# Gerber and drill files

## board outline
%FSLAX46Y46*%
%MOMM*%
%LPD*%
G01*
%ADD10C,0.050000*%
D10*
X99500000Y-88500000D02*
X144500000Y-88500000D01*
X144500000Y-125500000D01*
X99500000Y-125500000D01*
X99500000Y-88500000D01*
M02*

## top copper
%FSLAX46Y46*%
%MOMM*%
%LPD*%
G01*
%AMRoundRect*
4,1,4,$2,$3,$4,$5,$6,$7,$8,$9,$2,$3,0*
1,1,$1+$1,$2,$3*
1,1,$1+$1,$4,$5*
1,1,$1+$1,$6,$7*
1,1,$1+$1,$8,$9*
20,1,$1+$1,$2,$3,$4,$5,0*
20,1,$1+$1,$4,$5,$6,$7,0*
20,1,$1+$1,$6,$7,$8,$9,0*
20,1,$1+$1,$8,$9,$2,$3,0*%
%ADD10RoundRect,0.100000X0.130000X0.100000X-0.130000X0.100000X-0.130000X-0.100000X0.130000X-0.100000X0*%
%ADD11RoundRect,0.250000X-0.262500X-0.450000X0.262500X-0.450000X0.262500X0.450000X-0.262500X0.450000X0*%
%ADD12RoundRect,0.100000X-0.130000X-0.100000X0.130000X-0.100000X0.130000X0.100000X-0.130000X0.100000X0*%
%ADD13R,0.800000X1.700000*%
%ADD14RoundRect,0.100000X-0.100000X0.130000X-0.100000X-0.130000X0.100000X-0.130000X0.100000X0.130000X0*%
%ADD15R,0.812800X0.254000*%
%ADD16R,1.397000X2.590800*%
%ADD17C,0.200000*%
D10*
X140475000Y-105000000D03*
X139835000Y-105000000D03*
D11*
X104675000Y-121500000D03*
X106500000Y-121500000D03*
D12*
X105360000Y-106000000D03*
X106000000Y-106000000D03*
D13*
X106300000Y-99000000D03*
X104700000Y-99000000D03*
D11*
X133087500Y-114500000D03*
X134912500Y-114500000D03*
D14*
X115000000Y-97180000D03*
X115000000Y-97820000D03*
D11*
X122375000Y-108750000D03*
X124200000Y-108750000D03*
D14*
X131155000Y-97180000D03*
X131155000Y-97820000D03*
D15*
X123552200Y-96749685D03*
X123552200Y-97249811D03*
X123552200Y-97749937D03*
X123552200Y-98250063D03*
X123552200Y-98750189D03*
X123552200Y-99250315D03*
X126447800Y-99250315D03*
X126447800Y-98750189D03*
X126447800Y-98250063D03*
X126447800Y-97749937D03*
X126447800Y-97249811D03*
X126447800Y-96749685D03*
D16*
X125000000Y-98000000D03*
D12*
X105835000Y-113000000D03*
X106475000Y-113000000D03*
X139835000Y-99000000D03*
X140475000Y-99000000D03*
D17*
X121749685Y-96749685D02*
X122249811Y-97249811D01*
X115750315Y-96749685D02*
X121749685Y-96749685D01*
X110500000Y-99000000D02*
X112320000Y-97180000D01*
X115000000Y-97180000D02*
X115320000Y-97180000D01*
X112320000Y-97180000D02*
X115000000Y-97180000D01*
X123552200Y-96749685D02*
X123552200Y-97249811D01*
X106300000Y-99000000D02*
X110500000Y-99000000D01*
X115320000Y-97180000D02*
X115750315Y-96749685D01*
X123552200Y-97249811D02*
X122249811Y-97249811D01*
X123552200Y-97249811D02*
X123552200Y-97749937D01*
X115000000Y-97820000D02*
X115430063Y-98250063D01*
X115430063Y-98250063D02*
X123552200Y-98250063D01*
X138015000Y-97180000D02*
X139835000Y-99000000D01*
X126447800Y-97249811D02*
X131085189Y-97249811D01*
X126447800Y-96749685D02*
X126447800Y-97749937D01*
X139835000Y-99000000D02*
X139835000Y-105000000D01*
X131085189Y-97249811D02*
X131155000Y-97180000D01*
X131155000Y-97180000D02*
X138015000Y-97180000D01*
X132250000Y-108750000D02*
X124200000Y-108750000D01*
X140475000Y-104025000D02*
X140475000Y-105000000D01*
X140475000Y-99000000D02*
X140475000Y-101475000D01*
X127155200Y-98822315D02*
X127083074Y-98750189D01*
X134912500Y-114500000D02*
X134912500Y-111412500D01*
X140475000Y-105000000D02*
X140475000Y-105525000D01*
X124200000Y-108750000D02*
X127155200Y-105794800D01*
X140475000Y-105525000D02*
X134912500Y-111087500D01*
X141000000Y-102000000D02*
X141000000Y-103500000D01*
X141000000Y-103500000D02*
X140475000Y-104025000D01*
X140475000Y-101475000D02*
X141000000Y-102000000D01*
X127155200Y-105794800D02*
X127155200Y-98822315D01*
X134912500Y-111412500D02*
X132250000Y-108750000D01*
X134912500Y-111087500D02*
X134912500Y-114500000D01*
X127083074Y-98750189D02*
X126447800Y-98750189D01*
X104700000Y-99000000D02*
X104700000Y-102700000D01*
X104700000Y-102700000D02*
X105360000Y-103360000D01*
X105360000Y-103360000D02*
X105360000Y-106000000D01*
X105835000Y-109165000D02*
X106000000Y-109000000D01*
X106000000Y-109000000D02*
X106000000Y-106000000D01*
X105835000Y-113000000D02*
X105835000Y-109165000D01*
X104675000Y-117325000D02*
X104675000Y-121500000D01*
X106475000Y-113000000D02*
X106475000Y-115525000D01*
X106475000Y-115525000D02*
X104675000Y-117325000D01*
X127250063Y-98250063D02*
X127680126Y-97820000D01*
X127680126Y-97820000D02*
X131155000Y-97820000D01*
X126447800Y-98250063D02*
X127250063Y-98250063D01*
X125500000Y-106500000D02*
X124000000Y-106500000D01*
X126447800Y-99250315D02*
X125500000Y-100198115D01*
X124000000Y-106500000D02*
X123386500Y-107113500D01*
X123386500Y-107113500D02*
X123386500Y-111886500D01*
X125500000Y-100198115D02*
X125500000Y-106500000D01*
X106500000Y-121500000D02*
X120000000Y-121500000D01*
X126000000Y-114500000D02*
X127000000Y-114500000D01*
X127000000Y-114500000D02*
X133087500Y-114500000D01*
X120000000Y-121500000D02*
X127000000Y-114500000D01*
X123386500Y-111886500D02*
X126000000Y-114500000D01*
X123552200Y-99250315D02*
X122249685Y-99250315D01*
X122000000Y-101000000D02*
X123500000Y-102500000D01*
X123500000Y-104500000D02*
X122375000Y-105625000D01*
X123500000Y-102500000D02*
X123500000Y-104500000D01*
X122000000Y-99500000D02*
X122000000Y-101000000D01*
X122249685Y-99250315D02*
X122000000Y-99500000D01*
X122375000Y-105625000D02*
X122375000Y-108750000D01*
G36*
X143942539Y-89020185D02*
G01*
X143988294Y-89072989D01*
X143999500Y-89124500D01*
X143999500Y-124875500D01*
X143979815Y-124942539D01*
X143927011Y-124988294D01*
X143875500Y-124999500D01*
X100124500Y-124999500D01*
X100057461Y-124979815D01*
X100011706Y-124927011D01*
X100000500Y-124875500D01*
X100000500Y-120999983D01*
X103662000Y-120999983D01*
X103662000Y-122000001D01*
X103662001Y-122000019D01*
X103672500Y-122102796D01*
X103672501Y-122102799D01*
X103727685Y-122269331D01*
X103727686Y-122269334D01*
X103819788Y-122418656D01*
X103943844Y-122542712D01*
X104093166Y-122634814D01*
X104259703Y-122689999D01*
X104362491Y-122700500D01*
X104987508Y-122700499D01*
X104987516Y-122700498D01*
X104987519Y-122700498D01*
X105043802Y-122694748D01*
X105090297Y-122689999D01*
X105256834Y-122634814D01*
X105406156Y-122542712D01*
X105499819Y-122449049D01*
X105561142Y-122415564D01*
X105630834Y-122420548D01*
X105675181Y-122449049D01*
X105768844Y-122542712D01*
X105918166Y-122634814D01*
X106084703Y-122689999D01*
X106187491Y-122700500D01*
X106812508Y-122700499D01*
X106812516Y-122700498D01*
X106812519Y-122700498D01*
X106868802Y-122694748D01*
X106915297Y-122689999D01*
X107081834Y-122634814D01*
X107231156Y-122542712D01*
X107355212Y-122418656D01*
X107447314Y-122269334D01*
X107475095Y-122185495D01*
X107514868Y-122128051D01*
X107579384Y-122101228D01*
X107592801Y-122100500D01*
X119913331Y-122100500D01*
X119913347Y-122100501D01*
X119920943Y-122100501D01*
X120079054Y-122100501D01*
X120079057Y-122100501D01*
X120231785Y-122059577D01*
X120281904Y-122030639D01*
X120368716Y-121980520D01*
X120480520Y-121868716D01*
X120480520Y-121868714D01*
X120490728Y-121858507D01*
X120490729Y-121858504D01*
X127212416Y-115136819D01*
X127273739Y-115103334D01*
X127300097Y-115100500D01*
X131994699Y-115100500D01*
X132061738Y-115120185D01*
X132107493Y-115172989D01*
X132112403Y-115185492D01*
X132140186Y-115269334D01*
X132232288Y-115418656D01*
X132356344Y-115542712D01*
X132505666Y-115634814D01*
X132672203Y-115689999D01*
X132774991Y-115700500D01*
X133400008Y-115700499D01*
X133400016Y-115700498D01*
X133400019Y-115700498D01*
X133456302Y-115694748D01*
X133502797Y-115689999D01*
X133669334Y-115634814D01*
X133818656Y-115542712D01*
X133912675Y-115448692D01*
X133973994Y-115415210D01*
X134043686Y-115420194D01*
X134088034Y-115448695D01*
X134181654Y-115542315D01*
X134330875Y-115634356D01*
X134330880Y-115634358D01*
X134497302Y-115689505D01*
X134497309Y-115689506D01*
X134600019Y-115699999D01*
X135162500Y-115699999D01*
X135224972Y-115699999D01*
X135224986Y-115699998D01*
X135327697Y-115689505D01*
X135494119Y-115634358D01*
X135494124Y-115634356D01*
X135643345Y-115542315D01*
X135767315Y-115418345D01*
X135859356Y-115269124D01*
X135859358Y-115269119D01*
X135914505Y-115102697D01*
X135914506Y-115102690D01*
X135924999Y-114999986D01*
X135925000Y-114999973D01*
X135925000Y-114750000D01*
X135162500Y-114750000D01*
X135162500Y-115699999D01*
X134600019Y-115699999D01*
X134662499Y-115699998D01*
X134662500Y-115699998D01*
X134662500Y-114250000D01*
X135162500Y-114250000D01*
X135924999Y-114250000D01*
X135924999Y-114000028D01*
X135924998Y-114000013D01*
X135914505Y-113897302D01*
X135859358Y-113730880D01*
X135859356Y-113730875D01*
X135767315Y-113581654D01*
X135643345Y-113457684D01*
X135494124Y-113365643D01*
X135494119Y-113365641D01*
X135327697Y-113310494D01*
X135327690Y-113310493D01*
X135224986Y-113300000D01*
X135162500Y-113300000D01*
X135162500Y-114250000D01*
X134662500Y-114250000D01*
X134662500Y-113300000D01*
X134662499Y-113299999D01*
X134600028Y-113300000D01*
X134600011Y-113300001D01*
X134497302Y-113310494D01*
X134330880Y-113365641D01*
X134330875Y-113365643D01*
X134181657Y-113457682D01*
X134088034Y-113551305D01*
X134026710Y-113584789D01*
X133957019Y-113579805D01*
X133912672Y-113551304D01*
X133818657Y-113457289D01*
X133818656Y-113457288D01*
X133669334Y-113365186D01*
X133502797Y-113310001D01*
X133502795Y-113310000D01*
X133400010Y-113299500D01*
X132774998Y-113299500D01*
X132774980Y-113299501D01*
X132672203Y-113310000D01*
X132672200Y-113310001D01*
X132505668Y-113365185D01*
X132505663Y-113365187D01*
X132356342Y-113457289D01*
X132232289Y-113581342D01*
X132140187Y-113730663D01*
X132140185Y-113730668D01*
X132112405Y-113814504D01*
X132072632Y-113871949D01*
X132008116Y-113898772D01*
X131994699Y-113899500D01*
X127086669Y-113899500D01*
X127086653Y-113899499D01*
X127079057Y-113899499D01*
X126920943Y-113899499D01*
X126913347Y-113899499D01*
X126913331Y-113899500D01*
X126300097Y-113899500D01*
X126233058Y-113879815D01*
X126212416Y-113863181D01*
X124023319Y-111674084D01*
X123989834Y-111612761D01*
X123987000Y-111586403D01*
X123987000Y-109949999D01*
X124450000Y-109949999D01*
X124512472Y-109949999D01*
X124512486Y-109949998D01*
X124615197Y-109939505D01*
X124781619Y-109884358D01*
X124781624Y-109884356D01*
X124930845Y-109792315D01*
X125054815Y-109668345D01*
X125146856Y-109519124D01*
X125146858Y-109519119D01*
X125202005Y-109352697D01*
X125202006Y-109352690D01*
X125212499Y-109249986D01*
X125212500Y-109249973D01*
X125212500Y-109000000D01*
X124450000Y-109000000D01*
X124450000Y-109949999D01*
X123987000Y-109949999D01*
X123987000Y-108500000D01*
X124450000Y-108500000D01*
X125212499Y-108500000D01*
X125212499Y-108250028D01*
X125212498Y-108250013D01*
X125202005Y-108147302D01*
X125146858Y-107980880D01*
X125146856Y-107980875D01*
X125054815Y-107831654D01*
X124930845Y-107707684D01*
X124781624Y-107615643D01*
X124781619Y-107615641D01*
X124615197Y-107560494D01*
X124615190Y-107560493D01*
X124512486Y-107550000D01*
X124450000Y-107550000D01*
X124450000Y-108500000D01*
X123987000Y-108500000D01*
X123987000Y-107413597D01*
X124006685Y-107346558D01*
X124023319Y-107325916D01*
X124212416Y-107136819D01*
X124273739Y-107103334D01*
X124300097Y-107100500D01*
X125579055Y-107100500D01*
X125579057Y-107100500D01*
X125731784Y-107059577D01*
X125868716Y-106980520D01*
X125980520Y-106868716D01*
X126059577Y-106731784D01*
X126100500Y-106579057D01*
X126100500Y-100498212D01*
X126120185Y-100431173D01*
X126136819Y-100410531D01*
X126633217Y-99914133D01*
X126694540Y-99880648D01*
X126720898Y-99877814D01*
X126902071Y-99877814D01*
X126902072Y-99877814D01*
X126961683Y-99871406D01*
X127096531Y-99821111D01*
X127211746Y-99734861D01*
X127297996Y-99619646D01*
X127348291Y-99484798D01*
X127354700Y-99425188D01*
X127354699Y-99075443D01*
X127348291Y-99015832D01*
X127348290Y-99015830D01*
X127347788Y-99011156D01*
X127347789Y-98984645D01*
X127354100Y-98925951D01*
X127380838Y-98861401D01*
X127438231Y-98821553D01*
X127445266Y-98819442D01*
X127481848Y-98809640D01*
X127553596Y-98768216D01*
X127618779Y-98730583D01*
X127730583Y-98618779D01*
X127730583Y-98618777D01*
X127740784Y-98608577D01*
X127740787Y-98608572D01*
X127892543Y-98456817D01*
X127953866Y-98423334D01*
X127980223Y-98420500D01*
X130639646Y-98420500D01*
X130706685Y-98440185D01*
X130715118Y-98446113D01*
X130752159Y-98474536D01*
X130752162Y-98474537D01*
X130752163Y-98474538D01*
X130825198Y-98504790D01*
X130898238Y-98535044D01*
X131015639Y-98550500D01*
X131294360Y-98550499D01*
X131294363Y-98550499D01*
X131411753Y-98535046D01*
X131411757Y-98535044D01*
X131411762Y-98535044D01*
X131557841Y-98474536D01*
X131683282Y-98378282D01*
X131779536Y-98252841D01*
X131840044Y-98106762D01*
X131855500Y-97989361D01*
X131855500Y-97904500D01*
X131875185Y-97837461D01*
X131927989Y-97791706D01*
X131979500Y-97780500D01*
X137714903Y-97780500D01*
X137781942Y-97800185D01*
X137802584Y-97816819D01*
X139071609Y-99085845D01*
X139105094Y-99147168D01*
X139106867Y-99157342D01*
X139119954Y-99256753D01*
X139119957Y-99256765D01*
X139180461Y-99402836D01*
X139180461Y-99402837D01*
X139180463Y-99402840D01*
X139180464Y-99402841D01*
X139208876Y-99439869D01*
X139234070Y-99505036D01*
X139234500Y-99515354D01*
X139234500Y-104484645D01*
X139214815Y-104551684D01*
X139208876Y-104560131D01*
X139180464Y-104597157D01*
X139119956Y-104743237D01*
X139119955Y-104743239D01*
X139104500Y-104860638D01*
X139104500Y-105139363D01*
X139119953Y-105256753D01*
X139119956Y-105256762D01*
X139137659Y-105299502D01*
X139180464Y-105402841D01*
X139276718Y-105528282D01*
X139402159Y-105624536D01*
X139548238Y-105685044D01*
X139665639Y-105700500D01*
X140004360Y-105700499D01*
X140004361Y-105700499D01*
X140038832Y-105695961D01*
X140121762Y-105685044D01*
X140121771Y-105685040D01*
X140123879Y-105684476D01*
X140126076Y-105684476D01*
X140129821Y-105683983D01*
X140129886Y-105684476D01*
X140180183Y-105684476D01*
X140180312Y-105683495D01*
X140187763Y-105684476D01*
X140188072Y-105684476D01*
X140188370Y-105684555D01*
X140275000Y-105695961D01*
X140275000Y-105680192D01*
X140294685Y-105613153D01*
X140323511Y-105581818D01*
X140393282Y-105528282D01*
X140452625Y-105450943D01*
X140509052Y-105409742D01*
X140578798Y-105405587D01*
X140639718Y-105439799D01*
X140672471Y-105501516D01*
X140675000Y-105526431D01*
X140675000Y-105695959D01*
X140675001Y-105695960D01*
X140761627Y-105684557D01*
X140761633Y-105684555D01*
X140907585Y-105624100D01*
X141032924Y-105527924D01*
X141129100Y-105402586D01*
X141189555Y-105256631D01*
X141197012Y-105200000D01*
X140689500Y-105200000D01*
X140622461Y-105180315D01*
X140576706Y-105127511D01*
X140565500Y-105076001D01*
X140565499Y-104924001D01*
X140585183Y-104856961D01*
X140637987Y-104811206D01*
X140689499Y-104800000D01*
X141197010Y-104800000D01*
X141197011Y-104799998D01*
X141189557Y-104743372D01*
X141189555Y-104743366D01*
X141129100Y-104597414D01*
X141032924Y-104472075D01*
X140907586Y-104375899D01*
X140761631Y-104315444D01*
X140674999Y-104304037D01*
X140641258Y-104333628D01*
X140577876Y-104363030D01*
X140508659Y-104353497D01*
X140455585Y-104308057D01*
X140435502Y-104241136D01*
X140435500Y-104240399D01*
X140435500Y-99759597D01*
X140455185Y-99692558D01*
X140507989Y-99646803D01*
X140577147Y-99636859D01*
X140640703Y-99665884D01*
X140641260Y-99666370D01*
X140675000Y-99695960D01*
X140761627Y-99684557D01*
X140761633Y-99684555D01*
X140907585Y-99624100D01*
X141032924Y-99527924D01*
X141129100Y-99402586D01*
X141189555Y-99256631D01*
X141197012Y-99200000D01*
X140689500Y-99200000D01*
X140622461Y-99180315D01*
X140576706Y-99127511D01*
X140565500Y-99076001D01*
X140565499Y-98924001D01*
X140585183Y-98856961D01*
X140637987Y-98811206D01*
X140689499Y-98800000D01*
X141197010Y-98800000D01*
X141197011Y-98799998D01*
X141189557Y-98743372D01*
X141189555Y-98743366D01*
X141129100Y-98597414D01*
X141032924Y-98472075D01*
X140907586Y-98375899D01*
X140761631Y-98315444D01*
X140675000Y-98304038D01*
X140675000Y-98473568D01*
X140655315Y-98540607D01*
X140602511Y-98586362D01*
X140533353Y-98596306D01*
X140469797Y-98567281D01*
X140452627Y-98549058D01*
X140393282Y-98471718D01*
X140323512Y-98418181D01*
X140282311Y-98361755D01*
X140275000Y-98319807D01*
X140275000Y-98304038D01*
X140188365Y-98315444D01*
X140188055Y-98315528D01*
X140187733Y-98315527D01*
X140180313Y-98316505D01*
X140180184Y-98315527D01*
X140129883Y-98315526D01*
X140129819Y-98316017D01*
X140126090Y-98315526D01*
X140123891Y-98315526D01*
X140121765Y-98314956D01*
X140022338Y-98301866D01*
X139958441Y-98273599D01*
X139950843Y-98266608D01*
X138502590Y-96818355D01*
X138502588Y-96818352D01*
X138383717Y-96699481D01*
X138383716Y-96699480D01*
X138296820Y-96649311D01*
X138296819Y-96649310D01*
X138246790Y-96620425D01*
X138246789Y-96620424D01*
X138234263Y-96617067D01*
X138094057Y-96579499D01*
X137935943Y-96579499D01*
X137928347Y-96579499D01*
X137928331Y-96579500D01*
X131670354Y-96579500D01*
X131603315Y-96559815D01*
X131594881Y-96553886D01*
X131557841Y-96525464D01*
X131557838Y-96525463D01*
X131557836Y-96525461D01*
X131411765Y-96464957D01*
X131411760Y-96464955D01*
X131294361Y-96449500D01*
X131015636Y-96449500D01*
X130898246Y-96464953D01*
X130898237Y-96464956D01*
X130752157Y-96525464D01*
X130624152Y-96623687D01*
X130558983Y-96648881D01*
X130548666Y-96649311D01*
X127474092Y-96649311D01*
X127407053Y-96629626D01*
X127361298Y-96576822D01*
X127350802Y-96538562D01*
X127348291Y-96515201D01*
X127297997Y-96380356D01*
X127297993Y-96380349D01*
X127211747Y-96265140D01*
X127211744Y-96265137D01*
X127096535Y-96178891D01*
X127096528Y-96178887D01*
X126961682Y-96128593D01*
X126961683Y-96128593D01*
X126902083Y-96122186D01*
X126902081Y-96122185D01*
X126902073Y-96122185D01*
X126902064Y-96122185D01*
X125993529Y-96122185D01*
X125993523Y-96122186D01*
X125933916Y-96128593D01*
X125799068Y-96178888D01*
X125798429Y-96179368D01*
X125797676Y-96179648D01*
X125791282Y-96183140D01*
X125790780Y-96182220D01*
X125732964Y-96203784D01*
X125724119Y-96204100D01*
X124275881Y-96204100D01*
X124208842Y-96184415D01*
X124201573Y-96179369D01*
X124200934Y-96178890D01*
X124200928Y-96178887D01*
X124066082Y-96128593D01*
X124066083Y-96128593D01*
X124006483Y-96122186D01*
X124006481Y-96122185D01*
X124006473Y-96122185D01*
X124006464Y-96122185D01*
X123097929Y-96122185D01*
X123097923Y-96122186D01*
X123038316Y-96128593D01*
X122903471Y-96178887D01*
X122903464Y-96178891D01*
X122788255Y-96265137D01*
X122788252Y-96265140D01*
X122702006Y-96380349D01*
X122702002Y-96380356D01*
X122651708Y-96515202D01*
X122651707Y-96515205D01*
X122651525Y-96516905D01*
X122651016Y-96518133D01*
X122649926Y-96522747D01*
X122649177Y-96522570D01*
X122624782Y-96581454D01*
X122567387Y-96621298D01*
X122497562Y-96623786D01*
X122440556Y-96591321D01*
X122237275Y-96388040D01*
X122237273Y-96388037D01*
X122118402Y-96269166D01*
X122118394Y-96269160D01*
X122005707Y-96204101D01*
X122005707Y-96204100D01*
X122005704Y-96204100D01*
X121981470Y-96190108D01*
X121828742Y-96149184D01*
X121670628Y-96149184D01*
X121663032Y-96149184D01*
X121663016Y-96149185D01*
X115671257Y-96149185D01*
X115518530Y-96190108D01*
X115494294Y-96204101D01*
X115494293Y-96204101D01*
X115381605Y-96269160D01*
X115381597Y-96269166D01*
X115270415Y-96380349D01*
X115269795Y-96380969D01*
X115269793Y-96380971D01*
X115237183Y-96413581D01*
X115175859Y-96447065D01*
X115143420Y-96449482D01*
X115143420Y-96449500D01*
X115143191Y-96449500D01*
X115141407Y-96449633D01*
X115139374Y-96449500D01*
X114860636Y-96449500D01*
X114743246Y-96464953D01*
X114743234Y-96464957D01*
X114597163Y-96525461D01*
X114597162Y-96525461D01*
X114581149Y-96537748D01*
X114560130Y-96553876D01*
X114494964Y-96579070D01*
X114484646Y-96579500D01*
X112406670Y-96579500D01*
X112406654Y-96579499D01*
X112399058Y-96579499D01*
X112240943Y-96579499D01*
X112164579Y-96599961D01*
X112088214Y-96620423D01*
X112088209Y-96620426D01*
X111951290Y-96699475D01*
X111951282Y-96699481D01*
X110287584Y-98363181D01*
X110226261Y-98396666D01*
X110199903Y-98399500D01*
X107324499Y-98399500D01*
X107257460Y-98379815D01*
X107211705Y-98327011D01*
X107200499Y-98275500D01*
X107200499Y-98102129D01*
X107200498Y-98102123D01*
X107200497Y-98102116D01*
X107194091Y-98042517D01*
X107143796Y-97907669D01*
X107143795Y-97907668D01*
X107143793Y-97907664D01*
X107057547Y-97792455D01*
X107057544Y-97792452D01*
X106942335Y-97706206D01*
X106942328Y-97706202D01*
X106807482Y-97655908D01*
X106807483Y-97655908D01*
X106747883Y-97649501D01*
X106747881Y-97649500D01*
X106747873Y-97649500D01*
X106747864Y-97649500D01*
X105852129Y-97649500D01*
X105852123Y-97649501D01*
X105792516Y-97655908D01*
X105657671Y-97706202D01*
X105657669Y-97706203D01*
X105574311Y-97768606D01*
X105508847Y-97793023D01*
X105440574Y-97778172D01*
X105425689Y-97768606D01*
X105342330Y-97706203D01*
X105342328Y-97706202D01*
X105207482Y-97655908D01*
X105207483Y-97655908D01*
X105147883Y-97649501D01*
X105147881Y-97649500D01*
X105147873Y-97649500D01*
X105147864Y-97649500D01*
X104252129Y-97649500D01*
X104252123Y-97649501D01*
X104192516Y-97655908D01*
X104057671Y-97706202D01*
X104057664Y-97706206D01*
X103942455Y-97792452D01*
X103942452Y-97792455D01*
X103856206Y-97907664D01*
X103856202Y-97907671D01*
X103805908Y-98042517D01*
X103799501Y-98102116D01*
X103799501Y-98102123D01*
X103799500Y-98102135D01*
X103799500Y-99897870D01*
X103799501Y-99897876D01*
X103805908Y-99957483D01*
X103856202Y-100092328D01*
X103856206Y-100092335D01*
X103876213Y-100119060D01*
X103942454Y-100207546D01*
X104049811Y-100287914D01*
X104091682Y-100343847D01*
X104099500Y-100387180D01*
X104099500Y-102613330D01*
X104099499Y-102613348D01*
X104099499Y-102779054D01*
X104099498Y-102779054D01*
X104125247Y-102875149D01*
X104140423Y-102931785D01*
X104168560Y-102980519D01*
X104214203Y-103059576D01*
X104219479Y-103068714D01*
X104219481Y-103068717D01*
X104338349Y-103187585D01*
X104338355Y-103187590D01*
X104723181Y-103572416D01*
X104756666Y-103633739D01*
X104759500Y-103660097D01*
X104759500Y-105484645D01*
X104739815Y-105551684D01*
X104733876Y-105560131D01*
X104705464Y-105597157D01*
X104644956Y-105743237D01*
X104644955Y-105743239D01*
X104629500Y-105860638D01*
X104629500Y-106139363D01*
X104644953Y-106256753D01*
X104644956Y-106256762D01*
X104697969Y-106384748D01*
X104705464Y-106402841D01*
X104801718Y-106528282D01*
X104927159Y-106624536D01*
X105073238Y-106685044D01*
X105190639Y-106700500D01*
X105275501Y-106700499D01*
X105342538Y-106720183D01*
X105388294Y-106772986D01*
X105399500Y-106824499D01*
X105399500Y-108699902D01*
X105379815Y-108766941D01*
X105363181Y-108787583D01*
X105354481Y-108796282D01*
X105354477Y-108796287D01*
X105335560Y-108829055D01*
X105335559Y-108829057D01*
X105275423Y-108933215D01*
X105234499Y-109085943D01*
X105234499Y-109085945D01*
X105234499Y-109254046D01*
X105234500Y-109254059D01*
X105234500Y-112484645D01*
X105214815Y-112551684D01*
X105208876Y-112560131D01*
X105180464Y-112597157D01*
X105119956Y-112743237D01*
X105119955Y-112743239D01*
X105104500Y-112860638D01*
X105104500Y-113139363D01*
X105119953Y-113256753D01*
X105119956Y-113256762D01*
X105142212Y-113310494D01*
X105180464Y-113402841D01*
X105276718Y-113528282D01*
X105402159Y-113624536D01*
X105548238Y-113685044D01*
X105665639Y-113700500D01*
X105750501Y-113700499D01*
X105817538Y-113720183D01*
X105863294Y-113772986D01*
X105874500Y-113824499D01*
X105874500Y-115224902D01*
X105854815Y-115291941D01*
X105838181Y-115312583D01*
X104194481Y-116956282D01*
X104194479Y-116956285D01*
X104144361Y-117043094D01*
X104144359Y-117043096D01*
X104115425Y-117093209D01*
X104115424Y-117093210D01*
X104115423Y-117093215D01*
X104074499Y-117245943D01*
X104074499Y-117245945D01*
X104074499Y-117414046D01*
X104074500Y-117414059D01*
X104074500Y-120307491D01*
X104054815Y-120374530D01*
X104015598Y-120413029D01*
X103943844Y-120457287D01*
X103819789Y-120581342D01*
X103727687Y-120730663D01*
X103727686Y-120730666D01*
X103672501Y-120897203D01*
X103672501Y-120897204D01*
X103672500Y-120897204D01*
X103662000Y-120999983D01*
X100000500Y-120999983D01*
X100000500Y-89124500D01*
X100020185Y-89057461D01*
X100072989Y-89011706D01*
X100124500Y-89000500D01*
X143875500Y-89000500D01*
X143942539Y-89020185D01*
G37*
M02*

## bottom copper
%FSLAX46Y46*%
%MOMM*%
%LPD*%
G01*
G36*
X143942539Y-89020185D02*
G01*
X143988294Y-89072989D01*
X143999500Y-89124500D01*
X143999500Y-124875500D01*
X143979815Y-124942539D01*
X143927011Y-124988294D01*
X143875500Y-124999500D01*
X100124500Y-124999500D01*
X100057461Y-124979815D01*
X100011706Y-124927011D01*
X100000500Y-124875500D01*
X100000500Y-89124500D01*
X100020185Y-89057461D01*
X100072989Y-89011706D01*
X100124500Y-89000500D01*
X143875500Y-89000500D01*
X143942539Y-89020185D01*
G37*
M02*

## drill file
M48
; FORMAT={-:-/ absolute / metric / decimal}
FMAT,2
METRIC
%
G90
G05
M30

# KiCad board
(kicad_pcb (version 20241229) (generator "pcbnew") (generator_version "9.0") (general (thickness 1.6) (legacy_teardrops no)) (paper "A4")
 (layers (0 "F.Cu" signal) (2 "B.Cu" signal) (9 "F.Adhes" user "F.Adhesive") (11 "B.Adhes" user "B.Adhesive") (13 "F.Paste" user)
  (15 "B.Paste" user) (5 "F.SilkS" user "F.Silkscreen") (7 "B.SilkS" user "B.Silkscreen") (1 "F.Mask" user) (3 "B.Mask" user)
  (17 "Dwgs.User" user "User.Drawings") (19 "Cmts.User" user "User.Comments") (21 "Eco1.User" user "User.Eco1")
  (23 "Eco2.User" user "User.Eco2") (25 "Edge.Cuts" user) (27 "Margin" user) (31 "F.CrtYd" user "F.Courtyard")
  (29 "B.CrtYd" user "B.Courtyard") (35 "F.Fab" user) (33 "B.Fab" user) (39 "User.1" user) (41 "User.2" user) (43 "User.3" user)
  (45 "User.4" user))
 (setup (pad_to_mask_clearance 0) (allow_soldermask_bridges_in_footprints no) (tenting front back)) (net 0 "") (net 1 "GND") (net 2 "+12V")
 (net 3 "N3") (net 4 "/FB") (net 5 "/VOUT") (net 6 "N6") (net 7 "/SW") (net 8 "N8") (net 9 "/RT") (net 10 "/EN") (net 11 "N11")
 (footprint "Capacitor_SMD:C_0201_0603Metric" (layer "F.Cu") (at 140.155 105 180)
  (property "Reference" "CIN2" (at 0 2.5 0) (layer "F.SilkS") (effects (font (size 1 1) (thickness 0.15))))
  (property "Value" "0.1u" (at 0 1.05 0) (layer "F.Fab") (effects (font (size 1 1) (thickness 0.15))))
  (pad "" smd roundrect (at -0.345 0 180) (size 0.318 0.36) (layers "F.Paste") (roundrect_rratio 0.25))
  (pad "" smd roundrect (at 0.345 0 180) (size 0.318 0.36) (layers "F.Paste") (roundrect_rratio 0.25))
  (pad "1" smd roundrect (at -0.32 0 180) (size 0.46 0.4) (layers "F.Cu" "F.Mask") (roundrect_rratio 0.25) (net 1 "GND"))
  (pad "2" smd roundrect (at 0.32 0 180) (size 0.46 0.4) (layers "F.Cu" "F.Mask") (roundrect_rratio 0.25) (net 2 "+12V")))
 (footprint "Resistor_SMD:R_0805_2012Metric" (layer "F.Cu") (at 105.5875 121.5)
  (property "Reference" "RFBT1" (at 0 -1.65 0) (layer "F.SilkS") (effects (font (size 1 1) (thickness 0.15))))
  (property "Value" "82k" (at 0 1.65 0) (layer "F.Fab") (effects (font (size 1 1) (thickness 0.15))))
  (pad "1" smd roundrect (at -0.9125 0) (size 1.025 1.4) (layers "F.Cu" "F.Mask" "F.Paste") (roundrect_rratio 0.243902) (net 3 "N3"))
  (pad "2" smd roundrect (at 0.9125 0) (size 1.025 1.4) (layers "F.Cu" "F.Mask" "F.Paste") (roundrect_rratio 0.243902) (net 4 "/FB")))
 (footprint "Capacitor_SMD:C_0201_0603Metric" (layer "F.Cu") (at 105.68 106)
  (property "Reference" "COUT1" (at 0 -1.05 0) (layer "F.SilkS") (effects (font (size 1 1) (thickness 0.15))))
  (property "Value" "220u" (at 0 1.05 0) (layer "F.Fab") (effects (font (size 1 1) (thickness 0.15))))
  (pad "" smd roundrect (at -0.345 0) (size 0.318 0.36) (layers "F.Paste") (roundrect_rratio 0.25))
  (pad "" smd roundrect (at 0.345 0) (size 0.318 0.36) (layers "F.Paste") (roundrect_rratio 0.25))
  (pad "1" smd roundrect (at -0.32 0) (size 0.46 0.4) (layers "F.Cu" "F.Mask") (roundrect_rratio 0.25) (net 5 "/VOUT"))
  (pad "2" smd roundrect (at 0.32 0) (size 0.46 0.4) (layers "F.Cu" "F.Mask") (roundrect_rratio 0.25) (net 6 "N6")))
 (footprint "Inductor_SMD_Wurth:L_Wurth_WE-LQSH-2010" (layer "F.Cu") (at 105.5 99 180)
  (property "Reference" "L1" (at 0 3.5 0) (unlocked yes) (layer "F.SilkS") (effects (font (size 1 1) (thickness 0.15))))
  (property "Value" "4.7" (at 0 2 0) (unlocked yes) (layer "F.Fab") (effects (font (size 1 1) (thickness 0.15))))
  (pad "1" smd rect (at -0.8 0 180) (size 0.8 1.7) (layers "F.Cu" "F.Mask" "F.Paste") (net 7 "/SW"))
  (pad "2" smd rect (at 0.8 0 180) (size 0.8 1.7) (layers "F.Cu" "F.Mask" "F.Paste") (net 5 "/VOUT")))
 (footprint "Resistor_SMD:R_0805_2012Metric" (layer "F.Cu") (at 134 114.5)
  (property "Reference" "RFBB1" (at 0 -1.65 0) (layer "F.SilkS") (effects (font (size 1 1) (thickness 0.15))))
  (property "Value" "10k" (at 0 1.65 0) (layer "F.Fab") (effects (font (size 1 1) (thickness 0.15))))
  (pad "1" smd roundrect (at -0.9125 0) (size 1.025 1.4) (layers "F.Cu" "F.Mask" "F.Paste") (roundrect_rratio 0.243902) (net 4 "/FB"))
  (pad "2" smd roundrect (at 0.9125 0) (size 1.025 1.4) (layers "F.Cu" "F.Mask" "F.Paste") (roundrect_rratio 0.243902) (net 1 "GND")))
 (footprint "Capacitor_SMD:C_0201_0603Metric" (layer "F.Cu") (at 115 97.5 -90)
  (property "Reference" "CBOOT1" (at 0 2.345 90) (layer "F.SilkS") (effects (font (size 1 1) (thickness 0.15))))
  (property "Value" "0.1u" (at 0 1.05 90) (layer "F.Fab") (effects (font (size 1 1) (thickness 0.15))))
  (pad "" smd roundrect (at -0.345 0 270) (size 0.318 0.36) (layers "F.Paste") (roundrect_rratio 0.25))
  (pad "" smd roundrect (at 0.345 0 270) (size 0.318 0.36) (layers "F.Paste") (roundrect_rratio 0.25))
  (pad "1" smd roundrect (at -0.32 0 270) (size 0.46 0.4) (layers "F.Cu" "F.Mask") (roundrect_rratio 0.25) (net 7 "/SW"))
  (pad "2" smd roundrect (at 0.32 0 270) (size 0.46 0.4) (layers "F.Cu" "F.Mask") (roundrect_rratio 0.25) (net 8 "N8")))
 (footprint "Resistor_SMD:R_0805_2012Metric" (layer "F.Cu") (at 123.2875 108.75)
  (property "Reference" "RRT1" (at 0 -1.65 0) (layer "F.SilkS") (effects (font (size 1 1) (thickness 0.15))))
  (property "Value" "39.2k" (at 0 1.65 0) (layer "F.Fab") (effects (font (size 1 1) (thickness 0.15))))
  (pad "1" smd roundrect (at -0.9125 0) (size 1.025 1.4) (layers "F.Cu" "F.Mask" "F.Paste") (roundrect_rratio 0.243902) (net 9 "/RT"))
  (pad "2" smd roundrect (at 0.9125 0) (size 1.025 1.4) (layers "F.Cu" "F.Mask" "F.Paste") (roundrect_rratio 0.243902) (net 1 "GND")))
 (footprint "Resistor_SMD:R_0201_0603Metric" (layer "F.Cu") (at 131.155 97.5 -90)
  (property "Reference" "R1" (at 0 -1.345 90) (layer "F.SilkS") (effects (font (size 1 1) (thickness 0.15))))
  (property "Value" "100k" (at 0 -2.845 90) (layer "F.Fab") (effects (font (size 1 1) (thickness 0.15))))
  (pad "" smd roundrect (at -0.345 0 270) (size 0.318 0.36) (layers "F.Paste") (roundrect_rratio 0.25))
  (pad "" smd roundrect (at 0.345 0 270) (size 0.318 0.36) (layers "F.Paste") (roundrect_rratio 0.25))
  (pad "1" smd roundrect (at -0.32 0 270) (size 0.46 0.4) (layers "F.Cu" "F.Mask") (roundrect_rratio 0.25) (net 2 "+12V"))
  (pad "2" smd roundrect (at 0.32 0 270) (size 0.46 0.4) (layers "F.Cu" "F.Mask") (roundrect_rratio 0.25) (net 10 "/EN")))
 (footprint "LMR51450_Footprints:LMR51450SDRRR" (layer "F.Cu") (at 125 98)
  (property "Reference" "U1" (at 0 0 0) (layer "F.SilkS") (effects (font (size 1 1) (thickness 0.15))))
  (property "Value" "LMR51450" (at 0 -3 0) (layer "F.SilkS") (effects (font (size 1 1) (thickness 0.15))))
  (pad "1" smd rect (at -1.4478 -1.250315) (size 0.8128 0.254) (layers "F.Cu" "F.Mask" "F.Paste") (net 7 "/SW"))
  (pad "2" smd rect (at -1.4478 -0.750189) (size 0.8128 0.254) (layers "F.Cu" "F.Mask" "F.Paste") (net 7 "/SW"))
  (pad "3" smd rect (at -1.4478 -0.250063) (size 0.8128 0.254) (layers "F.Cu" "F.Mask" "F.Paste") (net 7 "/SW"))
  (pad "4" smd rect (at -1.4478 0.250063) (size 0.8128 0.254) (layers "F.Cu" "F.Mask" "F.Paste") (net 8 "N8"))
  (pad "5" smd rect (at -1.4478 0.750189) (size 0.8128 0.254) (layers "F.Cu" "F.Mask" "F.Paste") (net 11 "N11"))
  (pad "6" smd rect (at -1.4478 1.250315) (size 0.8128 0.254) (layers "F.Cu" "F.Mask" "F.Paste") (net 9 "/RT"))
  (pad "7" smd rect (at 1.4478 1.250315) (size 0.8128 0.254) (layers "F.Cu" "F.Mask" "F.Paste") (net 4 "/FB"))
  (pad "8" smd rect (at 1.4478 0.750189) (size 0.8128 0.254) (layers "F.Cu" "F.Mask" "F.Paste") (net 1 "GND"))
  (pad "9" smd rect (at 1.4478 0.250063) (size 0.8128 0.254) (layers "F.Cu" "F.Mask" "F.Paste") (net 10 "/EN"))
  (pad "10" smd rect (at 1.4478 -0.250063) (size 0.8128 0.254) (layers "F.Cu" "F.Mask" "F.Paste") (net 2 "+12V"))
  (pad "11" smd rect (at 1.4478 -0.750189) (size 0.8128 0.254) (layers "F.Cu" "F.Mask" "F.Paste") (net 2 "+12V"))
  (pad "12" smd rect (at 1.4478 -1.250315) (size 0.8128 0.254) (layers "F.Cu" "F.Mask" "F.Paste") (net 2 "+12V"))
  (pad "13" smd rect (at 0 0) (size 1.397 2.5908) (layers "F.Cu" "F.Mask" "F.Paste")))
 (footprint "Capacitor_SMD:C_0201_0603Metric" (layer "F.Cu") (at 106.155 113)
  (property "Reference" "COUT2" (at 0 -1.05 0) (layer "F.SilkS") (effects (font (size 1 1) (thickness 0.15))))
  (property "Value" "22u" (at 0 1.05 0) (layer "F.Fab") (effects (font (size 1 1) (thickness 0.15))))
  (pad "" smd roundrect (at -0.345 0) (size 0.318 0.36) (layers "F.Paste") (roundrect_rratio 0.25))
  (pad "" smd roundrect (at 0.345 0) (size 0.318 0.36) (layers "F.Paste") (roundrect_rratio 0.25))
  (pad "1" smd roundrect (at -0.32 0) (size 0.46 0.4) (layers "F.Cu" "F.Mask") (roundrect_rratio 0.25) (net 6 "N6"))
  (pad "2" smd roundrect (at 0.32 0) (size 0.46 0.4) (layers "F.Cu" "F.Mask") (roundrect_rratio 0.25) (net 3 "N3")))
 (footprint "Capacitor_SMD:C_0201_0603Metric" (layer "F.Cu") (at 140.155 99)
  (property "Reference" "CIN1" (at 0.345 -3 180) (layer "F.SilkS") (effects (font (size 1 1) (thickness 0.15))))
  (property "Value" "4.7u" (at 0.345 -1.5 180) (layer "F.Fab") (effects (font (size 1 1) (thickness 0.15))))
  (pad "" smd roundrect (at -0.345 0) (size 0.318 0.36) (layers "F.Paste") (roundrect_rratio 0.25))
  (pad "" smd roundrect (at 0.345 0) (size 0.318 0.36) (layers "F.Paste") (roundrect_rratio 0.25))
  (pad "1" smd roundrect (at -0.32 0) (size 0.46 0.4) (layers "F.Cu" "F.Mask") (roundrect_rratio 0.25) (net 2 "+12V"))
  (pad "2" smd roundrect (at 0.32 0) (size 0.46 0.4) (layers "F.Cu" "F.Mask") (roundrect_rratio 0.25) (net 1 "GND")))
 (gr_rect (start 99.5 88.5) (end 144.5 125.5) (stroke (width 0.05) (type default)) (fill no) (layer "Edge.Cuts"))
 (segment (start 121.749685 96.749685) (end 122.249811 97.249811) (width 0.2) (layer "F.Cu") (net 7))
 (segment (start 115.750315 96.749685) (end 121.749685 96.749685) (width 0.2) (layer "F.Cu") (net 7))
 (segment (start 110.5 99) (end 112.32 97.18) (width 0.2) (layer "F.Cu") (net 7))
 (segment (start 115 97.18) (end 115.32 97.18) (width 0.2) (layer "F.Cu") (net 7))
 (segment (start 112.32 97.18) (end 115 97.18) (width 0.2) (layer "F.Cu") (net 7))
 (segment (start 123.5522 96.749685) (end 123.5522 97.249811) (width 0.2) (layer "F.Cu") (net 7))
 (segment (start 106.3 99) (end 110.5 99) (width 0.2) (layer "F.Cu") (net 7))
 (segment (start 115.32 97.18) (end 115.750315 96.749685) (width 0.2) (layer "F.Cu") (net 7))
 (segment (start 123.5522 97.249811) (end 122.249811 97.249811) (width 0.2) (layer "F.Cu") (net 7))
 (segment (start 123.5522 97.249811) (end 123.5522 97.749937) (width 0.2) (layer "F.Cu") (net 7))
 (segment (start 115 97.82) (end 115.430063 98.250063) (width 0.2) (layer "F.Cu") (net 8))
 (segment (start 115.430063 98.250063) (end 123.5522 98.250063) (width 0.2) (layer "F.Cu") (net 8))
 (segment (start 138.015 97.18) (end 139.835 99) (width 0.2) (layer "F.Cu") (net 2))
 (segment (start 126.4478 97.249811) (end 131.085189 97.249811) (width 0.2) (layer "F.Cu") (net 2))
 (segment (start 126.4478 96.749685) (end 126.4478 97.749937) (width 0.2) (layer "F.Cu") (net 2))
 (segment (start 139.835 99) (end 139.835 105) (width 0.2) (layer "F.Cu") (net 2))
 (segment (start 131.085189 97.249811) (end 131.155 97.18) (width 0.2) (layer "F.Cu") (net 2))
 (segment (start 131.155 97.18) (end 138.015 97.18) (width 0.2) (layer "F.Cu") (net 2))
 (segment (start 132.25 108.75) (end 124.2 108.75) (width 0.2) (layer "F.Cu") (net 1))
 (segment (start 140.475 104.025) (end 140.475 105) (width 0.2) (layer "F.Cu") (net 1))
 (segment (start 140.475 99) (end 140.475 101.475) (width 0.2) (layer "F.Cu") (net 1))
 (segment (start 127.1552 98.822315) (end 127.083074 98.750189) (width 0.2) (layer "F.Cu") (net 1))
 (segment (start 134.9125 114.5) (end 134.9125 111.4125) (width 0.2) (layer "F.Cu") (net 1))
 (segment (start 140.475 105) (end 140.475 105.525) (width 0.2) (layer "F.Cu") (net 1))
 (segment (start 124.2 108.75) (end 127.1552 105.7948) (width 0.2) (layer "F.Cu") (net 1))
 (segment (start 140.475 105.525) (end 134.9125 111.0875) (width 0.2) (layer "F.Cu") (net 1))
 (segment (start 141 102) (end 141 103.5) (width 0.2) (layer "F.Cu") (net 1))
 (segment (start 141 103.5) (end 140.475 104.025) (width 0.2) (layer "F.Cu") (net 1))
 (segment (start 140.475 101.475) (end 141 102) (width 0.2) (layer "F.Cu") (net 1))
 (segment (start 127.1552 105.7948) (end 127.1552 98.822315) (width 0.2) (layer "F.Cu") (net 1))
 (segment (start 134.9125 111.4125) (end 132.25 108.75) (width 0.2) (layer "F.Cu") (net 1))
 (segment (start 134.9125 111.0875) (end 134.9125 114.5) (width 0.2) (layer "F.Cu") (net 1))
 (segment (start 127.083074 98.750189) (end 126.4478 98.750189) (width 0.2) (layer "F.Cu") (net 1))
 (segment (start 104.7 99) (end 104.7 102.7) (width 0.2) (layer "F.Cu") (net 5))
 (segment (start 104.7 102.7) (end 105.36 103.36) (width 0.2) (layer "F.Cu") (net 5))
 (segment (start 105.36 103.36) (end 105.36 106) (width 0.2) (layer "F.Cu") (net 5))
 (segment (start 105.835 109.165) (end 106 109) (width 0.2) (layer "F.Cu") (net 6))
 (segment (start 106 109) (end 106 106) (width 0.2) (layer "F.Cu") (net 6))
 (segment (start 105.835 113) (end 105.835 109.165) (width 0.2) (layer "F.Cu") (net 6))
 (segment (start 104.675 117.325) (end 104.675 121.5) (width 0.2) (layer "F.Cu") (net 3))
 (segment (start 106.475 113) (end 106.475 115.525) (width 0.2) (layer "F.Cu") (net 3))
 (segment (start 106.475 115.525) (end 104.675 117.325) (width 0.2) (layer "F.Cu") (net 3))
 (segment (start 127.250063 98.250063) (end 127.680126 97.82) (width 0.2) (layer "F.Cu") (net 10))
 (segment (start 127.680126 97.82) (end 131.155 97.82) (width 0.2) (layer "F.Cu") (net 10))
 (segment (start 126.4478 98.250063) (end 127.250063 98.250063) (width 0.2) (layer "F.Cu") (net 10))
 (segment (start 125.5 106.5) (end 124 106.5) (width 0.2) (layer "F.Cu") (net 4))
 (segment (start 126.4478 99.250315) (end 125.5 100.198115) (width 0.2) (layer "F.Cu") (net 4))
 (segment (start 124 106.5) (end 123.3865 107.1135) (width 0.2) (layer "F.Cu") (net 4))
 (segment (start 123.3865 107.1135) (end 123.3865 111.8865) (width 0.2) (layer "F.Cu") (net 4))
 (segment (start 125.5 100.198115) (end 125.5 106.5) (width 0.2) (layer "F.Cu") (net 4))
 (segment (start 106.5 121.5) (end 120 121.5) (width 0.2) (layer "F.Cu") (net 4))
 (segment (start 126 114.5) (end 127 114.5) (width 0.2) (layer "F.Cu") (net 4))
 (segment (start 127 114.5) (end 133.0875 114.5) (width 0.2) (layer "F.Cu") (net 4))
 (segment (start 120 121.5) (end 127 114.5) (width 0.2) (layer "F.Cu") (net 4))
 (segment (start 123.3865 111.8865) (end 126 114.5) (width 0.2) (layer "F.Cu") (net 4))
 (segment (start 123.5522 99.250315) (end 122.249685 99.250315) (width 0.2) (layer "F.Cu") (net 9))
 (segment (start 122 101) (end 123.5 102.5) (width 0.2) (layer "F.Cu") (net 9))
 (segment (start 123.5 104.5) (end 122.375 105.625) (width 0.2) (layer "F.Cu") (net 9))
 (segment (start 123.5 102.5) (end 123.5 104.5) (width 0.2) (layer "F.Cu") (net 9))
 (segment (start 122 99.5) (end 122 101) (width 0.2) (layer "F.Cu") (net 9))
 (segment (start 122.249685 99.250315) (end 122 99.5) (width 0.2) (layer "F.Cu") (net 9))
 (segment (start 122.375 105.625) (end 122.375 108.75) (width 0.2) (layer "F.Cu") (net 9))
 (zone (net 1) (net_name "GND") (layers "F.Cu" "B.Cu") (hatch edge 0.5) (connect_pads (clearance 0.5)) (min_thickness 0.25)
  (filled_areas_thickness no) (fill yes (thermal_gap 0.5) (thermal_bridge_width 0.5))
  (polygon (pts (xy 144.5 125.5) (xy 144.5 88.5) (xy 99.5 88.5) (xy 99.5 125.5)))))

